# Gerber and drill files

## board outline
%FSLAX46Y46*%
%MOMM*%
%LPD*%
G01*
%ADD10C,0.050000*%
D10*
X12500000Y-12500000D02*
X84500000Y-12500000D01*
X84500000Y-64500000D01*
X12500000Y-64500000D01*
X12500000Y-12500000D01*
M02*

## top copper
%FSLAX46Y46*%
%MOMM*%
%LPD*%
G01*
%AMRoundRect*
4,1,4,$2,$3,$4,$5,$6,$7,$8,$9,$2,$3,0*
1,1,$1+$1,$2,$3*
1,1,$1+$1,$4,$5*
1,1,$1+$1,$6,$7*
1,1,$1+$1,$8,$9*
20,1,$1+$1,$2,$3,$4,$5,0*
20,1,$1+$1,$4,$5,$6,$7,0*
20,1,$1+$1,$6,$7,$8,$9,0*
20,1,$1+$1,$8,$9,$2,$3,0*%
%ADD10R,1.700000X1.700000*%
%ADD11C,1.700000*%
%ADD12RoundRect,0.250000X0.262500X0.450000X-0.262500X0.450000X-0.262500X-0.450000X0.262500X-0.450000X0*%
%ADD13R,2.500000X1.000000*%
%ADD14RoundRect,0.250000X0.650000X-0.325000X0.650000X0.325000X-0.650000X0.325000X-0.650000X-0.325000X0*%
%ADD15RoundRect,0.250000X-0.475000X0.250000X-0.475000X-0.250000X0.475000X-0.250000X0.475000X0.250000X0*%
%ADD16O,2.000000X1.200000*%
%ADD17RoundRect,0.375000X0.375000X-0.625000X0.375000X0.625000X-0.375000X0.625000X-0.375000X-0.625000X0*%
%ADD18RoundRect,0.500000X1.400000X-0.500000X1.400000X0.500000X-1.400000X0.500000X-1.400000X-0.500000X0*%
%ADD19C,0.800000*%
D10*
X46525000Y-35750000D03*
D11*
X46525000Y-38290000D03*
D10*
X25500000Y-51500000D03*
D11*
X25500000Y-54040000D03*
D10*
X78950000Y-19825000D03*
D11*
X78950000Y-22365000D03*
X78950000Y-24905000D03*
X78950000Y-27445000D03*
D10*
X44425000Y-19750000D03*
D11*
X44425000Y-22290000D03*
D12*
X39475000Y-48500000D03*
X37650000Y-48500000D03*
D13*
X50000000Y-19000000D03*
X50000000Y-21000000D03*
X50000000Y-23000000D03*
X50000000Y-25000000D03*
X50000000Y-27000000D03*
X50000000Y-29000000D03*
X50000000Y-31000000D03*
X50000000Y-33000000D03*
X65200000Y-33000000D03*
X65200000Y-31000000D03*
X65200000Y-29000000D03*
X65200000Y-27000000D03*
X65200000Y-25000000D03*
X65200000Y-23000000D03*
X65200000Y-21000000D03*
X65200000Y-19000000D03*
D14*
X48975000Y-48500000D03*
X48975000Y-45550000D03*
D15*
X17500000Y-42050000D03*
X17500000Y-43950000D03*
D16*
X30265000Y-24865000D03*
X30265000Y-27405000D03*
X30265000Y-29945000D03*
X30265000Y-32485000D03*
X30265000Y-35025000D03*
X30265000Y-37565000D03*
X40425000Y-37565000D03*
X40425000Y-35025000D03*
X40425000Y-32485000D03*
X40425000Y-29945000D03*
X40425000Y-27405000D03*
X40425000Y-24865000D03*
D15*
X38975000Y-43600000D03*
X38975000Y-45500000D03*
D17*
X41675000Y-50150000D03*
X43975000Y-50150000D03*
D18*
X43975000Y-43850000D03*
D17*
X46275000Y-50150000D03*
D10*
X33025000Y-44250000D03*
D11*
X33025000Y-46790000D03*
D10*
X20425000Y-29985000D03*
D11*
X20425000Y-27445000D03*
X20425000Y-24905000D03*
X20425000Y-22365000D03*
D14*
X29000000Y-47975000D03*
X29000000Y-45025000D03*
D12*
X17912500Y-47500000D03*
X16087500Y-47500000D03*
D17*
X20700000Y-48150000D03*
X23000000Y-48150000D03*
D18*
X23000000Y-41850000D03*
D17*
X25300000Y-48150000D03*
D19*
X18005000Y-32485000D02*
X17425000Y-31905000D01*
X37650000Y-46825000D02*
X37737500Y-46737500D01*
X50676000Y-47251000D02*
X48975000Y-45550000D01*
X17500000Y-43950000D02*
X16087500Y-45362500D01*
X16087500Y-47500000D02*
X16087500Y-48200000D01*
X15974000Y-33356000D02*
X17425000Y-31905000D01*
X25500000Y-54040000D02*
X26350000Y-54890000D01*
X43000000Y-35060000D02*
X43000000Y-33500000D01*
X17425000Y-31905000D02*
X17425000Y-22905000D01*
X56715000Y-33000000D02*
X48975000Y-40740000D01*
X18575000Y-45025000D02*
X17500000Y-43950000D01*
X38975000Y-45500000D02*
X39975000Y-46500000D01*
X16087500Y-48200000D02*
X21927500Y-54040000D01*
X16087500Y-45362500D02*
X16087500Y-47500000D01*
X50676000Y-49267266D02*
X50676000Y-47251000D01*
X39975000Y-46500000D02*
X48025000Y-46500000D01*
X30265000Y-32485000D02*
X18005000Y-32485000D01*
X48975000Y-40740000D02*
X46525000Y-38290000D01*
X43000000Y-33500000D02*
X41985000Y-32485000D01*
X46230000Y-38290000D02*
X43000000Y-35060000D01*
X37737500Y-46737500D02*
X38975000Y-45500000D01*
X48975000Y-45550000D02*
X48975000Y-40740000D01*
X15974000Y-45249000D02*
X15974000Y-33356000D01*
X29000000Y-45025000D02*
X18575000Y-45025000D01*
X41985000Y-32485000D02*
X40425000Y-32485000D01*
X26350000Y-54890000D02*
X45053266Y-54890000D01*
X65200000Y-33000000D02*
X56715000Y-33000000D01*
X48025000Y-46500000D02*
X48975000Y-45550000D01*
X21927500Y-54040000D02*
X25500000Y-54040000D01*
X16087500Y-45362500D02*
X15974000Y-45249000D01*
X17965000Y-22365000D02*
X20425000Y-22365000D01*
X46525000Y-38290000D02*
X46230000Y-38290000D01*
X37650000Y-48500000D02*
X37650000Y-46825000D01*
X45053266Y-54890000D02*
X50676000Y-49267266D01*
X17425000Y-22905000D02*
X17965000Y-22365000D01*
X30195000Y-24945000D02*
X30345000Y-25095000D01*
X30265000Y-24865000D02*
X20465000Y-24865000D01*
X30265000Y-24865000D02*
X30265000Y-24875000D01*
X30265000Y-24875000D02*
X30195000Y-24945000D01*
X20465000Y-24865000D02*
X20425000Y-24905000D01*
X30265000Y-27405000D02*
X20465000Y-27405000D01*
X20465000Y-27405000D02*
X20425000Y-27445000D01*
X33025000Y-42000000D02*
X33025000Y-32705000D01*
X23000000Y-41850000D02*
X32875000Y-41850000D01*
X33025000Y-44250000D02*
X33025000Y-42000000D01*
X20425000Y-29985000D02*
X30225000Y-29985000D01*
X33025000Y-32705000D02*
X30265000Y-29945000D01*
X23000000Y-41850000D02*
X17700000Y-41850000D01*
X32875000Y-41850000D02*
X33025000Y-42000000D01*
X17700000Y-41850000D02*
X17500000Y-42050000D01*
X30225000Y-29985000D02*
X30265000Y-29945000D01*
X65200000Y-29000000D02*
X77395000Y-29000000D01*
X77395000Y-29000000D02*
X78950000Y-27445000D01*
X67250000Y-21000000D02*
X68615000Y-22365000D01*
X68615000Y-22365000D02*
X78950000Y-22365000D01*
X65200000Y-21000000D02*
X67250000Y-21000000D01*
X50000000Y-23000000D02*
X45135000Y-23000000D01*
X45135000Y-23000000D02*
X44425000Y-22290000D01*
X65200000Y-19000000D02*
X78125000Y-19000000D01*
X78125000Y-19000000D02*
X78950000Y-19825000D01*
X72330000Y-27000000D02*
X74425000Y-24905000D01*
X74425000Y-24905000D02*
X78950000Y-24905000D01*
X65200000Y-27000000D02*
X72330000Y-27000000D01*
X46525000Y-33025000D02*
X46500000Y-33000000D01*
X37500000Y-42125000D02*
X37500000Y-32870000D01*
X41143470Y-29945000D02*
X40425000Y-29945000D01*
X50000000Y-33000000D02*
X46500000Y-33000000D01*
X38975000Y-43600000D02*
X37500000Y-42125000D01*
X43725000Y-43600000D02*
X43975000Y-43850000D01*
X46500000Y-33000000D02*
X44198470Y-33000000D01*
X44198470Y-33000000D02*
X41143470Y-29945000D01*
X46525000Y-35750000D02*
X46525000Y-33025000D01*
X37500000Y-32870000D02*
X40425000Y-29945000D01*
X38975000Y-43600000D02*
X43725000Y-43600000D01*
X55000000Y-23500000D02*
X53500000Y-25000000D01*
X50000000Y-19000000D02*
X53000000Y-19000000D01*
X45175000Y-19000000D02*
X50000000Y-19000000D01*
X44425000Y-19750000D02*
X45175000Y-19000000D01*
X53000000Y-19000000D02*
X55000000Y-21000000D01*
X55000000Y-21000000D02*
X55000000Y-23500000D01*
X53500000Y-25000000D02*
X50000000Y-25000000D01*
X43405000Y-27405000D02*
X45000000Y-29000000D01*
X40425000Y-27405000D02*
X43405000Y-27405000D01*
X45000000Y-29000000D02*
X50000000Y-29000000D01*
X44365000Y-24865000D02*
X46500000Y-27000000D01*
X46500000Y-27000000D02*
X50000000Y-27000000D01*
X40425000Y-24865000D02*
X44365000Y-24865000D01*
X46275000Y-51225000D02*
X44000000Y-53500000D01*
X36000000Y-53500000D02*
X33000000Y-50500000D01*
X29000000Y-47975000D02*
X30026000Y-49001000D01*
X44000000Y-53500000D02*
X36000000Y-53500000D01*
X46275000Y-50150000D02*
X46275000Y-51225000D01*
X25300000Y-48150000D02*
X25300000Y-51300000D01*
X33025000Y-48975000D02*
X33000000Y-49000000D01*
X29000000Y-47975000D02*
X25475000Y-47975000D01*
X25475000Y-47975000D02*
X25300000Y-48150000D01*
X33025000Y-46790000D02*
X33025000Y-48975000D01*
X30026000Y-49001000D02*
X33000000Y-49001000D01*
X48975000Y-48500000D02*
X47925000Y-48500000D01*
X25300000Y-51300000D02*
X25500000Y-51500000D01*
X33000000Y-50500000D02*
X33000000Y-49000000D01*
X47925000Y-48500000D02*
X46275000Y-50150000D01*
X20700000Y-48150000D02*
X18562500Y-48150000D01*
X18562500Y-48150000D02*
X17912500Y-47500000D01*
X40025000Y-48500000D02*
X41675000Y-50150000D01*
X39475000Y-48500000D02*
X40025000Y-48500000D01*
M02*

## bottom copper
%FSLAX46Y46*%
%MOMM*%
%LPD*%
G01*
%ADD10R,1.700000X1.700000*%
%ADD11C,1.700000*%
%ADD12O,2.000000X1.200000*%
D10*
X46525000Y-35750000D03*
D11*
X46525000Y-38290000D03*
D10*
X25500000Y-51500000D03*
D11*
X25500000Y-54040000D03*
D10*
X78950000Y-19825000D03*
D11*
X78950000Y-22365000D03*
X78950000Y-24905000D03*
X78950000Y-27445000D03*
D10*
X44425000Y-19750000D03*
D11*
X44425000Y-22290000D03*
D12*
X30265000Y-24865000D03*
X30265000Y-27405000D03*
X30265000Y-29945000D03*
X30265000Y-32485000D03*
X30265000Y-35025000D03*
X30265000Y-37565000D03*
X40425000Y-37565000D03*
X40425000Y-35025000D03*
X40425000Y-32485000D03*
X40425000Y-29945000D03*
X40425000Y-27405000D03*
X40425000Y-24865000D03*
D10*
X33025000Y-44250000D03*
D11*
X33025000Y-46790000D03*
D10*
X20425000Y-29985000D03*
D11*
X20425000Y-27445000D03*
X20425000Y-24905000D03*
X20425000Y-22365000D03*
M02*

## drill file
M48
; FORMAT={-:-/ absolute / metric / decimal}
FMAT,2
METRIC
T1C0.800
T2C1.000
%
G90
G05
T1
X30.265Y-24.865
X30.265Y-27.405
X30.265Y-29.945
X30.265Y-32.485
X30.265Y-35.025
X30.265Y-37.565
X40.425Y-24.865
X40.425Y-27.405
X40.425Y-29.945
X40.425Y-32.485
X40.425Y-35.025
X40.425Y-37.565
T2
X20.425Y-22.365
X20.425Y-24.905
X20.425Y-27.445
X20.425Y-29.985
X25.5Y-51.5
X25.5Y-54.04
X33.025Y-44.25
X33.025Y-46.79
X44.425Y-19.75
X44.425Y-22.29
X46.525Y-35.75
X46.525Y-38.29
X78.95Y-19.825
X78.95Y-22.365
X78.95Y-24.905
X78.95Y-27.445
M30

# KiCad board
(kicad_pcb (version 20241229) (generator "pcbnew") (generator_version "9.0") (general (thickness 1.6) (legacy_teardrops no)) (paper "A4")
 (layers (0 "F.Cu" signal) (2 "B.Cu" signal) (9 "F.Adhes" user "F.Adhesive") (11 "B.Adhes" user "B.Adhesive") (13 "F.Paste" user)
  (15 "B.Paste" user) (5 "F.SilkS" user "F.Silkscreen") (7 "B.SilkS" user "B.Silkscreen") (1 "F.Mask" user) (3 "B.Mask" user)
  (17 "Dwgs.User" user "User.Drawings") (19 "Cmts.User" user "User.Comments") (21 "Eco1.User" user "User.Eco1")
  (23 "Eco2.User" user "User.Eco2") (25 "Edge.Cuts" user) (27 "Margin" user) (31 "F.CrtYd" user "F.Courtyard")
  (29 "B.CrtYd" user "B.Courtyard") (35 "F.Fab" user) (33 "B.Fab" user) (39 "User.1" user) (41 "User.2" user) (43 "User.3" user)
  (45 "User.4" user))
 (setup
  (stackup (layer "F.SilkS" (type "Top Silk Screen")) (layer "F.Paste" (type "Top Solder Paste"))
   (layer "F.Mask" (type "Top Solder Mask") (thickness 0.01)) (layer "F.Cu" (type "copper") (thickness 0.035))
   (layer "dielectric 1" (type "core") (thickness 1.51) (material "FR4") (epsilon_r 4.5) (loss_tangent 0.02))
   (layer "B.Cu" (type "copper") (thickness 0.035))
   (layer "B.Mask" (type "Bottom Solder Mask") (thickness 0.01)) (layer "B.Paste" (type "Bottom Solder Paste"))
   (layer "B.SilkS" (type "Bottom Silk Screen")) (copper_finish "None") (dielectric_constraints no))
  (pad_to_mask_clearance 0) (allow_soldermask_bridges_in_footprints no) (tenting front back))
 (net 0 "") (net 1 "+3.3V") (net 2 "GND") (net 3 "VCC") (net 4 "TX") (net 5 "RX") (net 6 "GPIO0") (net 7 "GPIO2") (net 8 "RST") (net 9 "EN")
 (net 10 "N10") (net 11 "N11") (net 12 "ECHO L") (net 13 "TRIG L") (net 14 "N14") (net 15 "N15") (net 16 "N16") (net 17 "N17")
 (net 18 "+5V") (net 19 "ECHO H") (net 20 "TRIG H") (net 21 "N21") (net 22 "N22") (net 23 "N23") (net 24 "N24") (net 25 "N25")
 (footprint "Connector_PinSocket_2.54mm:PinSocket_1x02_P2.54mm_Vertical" (layer "F.Cu") (at 46.525 35.75)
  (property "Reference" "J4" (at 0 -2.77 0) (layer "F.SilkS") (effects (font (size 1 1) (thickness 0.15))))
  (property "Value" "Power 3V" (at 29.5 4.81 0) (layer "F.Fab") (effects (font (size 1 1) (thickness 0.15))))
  (pad "1" thru_hole rect (at 0 0) (size 1.7 1.7) (drill 1) (layers "*.Cu" "*.Mask") (remove_unused_layers no) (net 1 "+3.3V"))
  (pad "2" thru_hole circle (at 0 2.54) (size 1.7 1.7) (drill 1) (layers "*.Cu" "*.Mask") (remove_unused_layers no) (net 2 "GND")))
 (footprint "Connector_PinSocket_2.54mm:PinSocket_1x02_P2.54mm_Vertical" (layer "F.Cu") (at 25.5 51.5)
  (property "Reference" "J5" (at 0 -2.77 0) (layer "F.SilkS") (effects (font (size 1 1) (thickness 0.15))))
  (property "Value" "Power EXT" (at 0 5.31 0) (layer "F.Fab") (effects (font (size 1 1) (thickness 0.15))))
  (pad "1" thru_hole rect (at 0 0) (size 1.7 1.7) (drill 1) (layers "*.Cu" "*.Mask") (remove_unused_layers no) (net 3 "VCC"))
  (pad "2" thru_hole circle (at 0 2.54) (size 1.7 1.7) (drill 1) (layers "*.Cu" "*.Mask") (remove_unused_layers no) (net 2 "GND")))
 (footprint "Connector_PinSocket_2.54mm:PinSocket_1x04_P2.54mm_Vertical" (layer "F.Cu") (at 78.95 19.825)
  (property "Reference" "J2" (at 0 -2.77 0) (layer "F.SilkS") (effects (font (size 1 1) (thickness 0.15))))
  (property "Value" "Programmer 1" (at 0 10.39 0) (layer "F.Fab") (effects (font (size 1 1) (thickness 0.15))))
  (pad "1" thru_hole rect (at 0 0) (size 1.7 1.7) (drill 1) (layers "*.Cu" "*.Mask") (remove_unused_layers no) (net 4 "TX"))
  (pad "2" thru_hole circle (at 0 2.54) (size 1.7 1.7) (drill 1) (layers "*.Cu" "*.Mask") (remove_unused_layers no) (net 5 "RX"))
  (pad "3" thru_hole circle (at 0 5.08) (size 1.7 1.7) (drill 1) (layers "*.Cu" "*.Mask") (remove_unused_layers no) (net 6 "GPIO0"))
  (pad "4" thru_hole circle (at 0 7.62) (size 1.7 1.7) (drill 1) (layers "*.Cu" "*.Mask") (remove_unused_layers no) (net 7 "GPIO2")))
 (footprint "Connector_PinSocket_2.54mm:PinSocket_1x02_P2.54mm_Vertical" (layer "F.Cu") (at 44.425 19.75)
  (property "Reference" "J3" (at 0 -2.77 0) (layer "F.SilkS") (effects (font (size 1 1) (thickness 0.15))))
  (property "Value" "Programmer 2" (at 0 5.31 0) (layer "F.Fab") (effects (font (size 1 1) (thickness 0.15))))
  (pad "1" thru_hole rect (at 0 0) (size 1.7 1.7) (drill 1) (layers "*.Cu" "*.Mask") (remove_unused_layers no) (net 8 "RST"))
  (pad "2" thru_hole circle (at 0 2.54) (size 1.7 1.7) (drill 1) (layers "*.Cu" "*.Mask") (remove_unused_layers no) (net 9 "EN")))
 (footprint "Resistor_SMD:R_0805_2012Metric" (layer "F.Cu") (at 38.5625 48.5 180)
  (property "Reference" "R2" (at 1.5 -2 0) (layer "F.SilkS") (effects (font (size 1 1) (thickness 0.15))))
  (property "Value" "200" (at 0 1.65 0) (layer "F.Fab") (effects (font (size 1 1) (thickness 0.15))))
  (pad "1" smd roundrect (at -0.9125 0 180) (size 1.025 1.4) (layers "F.Cu" "F.Mask" "F.Paste") (roundrect_rratio 0.243902) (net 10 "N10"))
  (pad "2" smd roundrect (at 0.9125 0 180) (size 1.025 1.4) (layers "F.Cu" "F.Mask" "F.Paste") (roundrect_rratio 0.243902) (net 2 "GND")))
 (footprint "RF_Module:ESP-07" (layer "F.Cu") (at 57.6 23.9)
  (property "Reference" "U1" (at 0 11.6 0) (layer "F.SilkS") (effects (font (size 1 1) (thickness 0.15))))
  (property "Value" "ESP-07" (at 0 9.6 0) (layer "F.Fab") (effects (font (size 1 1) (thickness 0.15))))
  (pad "1" smd rect (at -7.6 -4.9) (size 2.5 1) (layers "F.Cu" "F.Mask" "F.Paste") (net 8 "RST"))
  (pad "2" smd rect (at -7.6 -2.9) (size 2.5 1) (layers "F.Cu" "F.Mask" "F.Paste") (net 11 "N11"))
  (pad "3" smd rect (at -7.6 -0.9) (size 2.5 1) (layers "F.Cu" "F.Mask" "F.Paste") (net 9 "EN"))
  (pad "4" smd rect (at -7.6 1.1) (size 2.5 1) (layers "F.Cu" "F.Mask" "F.Paste") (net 8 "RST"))
  (pad "5" smd rect (at -7.6 3.1) (size 2.5 1) (layers "F.Cu" "F.Mask" "F.Paste") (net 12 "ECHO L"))
  (pad "6" smd rect (at -7.6 5.1) (size 2.5 1) (layers "F.Cu" "F.Mask" "F.Paste") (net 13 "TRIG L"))
  (pad "7" smd rect (at -7.6 7.1) (size 2.5 1) (layers "F.Cu" "F.Mask" "F.Paste") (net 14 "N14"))
  (pad "8" smd rect (at -7.6 9.1) (size 2.5 1) (layers "F.Cu" "F.Mask" "F.Paste") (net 1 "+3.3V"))
  (pad "9" smd rect (at 7.6 9.1) (size 2.5 1) (layers "F.Cu" "F.Mask" "F.Paste") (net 2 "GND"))
  (pad "10" smd rect (at 7.6 7.1) (size 2.5 1) (layers "F.Cu" "F.Mask" "F.Paste") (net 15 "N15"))
  (pad "11" smd rect (at 7.6 5.1) (size 2.5 1) (layers "F.Cu" "F.Mask" "F.Paste") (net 7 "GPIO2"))
  (pad "12" smd rect (at 7.6 3.1) (size 2.5 1) (layers "F.Cu" "F.Mask" "F.Paste") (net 6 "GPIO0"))
  (pad "13" smd rect (at 7.6 1.1) (size 2.5 1) (layers "F.Cu" "F.Mask" "F.Paste") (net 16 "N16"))
  (pad "14" smd rect (at 7.6 -0.9) (size 2.5 1) (layers "F.Cu" "F.Mask" "F.Paste") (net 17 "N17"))
  (pad "15" smd rect (at 7.6 -2.9) (size 2.5 1) (layers "F.Cu" "F.Mask" "F.Paste") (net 5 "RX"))
  (pad "16" smd rect (at 7.6 -4.9) (size 2.5 1) (layers "F.Cu" "F.Mask" "F.Paste") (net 4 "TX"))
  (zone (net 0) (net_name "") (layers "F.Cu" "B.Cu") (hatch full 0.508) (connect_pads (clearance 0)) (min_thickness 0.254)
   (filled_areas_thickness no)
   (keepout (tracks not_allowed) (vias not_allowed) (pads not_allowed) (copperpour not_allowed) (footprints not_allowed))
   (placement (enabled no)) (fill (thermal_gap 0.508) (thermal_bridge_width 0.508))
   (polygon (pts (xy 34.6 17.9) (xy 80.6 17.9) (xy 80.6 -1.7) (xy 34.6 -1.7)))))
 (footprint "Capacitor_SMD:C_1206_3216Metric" (layer "F.Cu") (at 48.975 47.025 90)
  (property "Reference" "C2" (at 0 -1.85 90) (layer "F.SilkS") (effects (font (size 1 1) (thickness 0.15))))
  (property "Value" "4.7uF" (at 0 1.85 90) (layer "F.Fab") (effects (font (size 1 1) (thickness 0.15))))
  (pad "1" smd roundrect (at -1.475 0 90) (size 1.15 1.8) (layers "F.Cu" "F.Mask" "F.Paste") (roundrect_rratio 0.217391) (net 3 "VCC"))
  (pad "2" smd roundrect (at 1.475 0 90) (size 1.15 1.8) (layers "F.Cu" "F.Mask" "F.Paste") (roundrect_rratio 0.217391) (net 2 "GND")))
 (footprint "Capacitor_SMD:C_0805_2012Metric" (layer "F.Cu") (at 17.5 43 -90)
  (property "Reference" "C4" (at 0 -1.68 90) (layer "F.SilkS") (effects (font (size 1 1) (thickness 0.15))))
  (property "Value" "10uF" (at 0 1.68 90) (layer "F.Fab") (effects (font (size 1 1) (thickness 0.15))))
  (pad "1" smd roundrect (at -0.95 0 270) (size 1 1.45) (layers "F.Cu" "F.Mask" "F.Paste") (roundrect_rratio 0.25) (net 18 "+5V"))
  (pad "2" smd roundrect (at 0.95 0 270) (size 1 1.45) (layers "F.Cu" "F.Mask" "F.Paste") (roundrect_rratio 0.25) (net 2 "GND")))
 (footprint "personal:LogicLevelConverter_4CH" (layer "F.Cu") (at 35.345 31.215 -90)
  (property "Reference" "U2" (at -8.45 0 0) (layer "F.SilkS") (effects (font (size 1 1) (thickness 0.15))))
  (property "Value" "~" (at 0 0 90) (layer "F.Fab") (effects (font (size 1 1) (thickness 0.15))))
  (pad "1" thru_hole oval (at -6.35 5.08 270) (size 1.2 2) (drill 0.8) (layers "*.Cu" "*.Mask") (remove_unused_layers no) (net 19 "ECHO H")
   (thermal_bridge_angle 45))
  (pad "2" thru_hole oval (at -3.81 5.08 270) (size 1.2 2) (drill 0.8) (layers "*.Cu" "*.Mask") (remove_unused_layers no) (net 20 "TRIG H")
   (thermal_bridge_angle 45))
  (pad "3" thru_hole oval (at -1.27 5.08 270) (size 1.2 2) (drill 0.8) (layers "*.Cu" "*.Mask") (remove_unused_layers no) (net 18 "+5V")
   (thermal_bridge_angle 45))
  (pad "4" thru_hole oval (at 1.27 5.08 270) (size 1.2 2) (drill 0.8) (layers "*.Cu" "*.Mask") (remove_unused_layers no) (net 2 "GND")
   (thermal_bridge_angle 45))
  (pad "5" thru_hole oval (at 3.81 5.08 270) (size 1.2 2) (drill 0.8) (layers "*.Cu" "*.Mask") (remove_unused_layers no) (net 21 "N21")
   (thermal_bridge_angle 45))
  (pad "6" thru_hole oval (at 6.35 5.08 270) (size 1.2 2) (drill 0.8) (layers "*.Cu" "*.Mask") (remove_unused_layers no) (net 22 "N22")
   (thermal_bridge_angle 45))
  (pad "7" thru_hole oval (at 6.35 -5.08 270) (size 1.2 2) (drill 0.8) (layers "*.Cu" "*.Mask") (remove_unused_layers no) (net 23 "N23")
   (thermal_bridge_angle 45))
  (pad "8" thru_hole oval (at 3.81 -5.08 270) (size 1.2 2) (drill 0.8) (layers "*.Cu" "*.Mask") (remove_unused_layers no) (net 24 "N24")
   (thermal_bridge_angle 45))
  (pad "9" thru_hole oval (at 1.27 -5.08 270) (size 1.2 2) (drill 0.8) (layers "*.Cu" "*.Mask") (remove_unused_layers no) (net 2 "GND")
   (thermal_bridge_angle 45))
  (pad "10" thru_hole oval (at -1.27 -5.08 270) (size 1.2 2) (drill 0.8) (layers "*.Cu" "*.Mask") (remove_unused_layers no) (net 1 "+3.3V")
   (thermal_bridge_angle 45))
  (pad "11" thru_hole oval (at -3.81 -5.08 270) (size 1.2 2) (drill 0.8) (layers "*.Cu" "*.Mask") (remove_unused_layers no)
   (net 13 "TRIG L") (thermal_bridge_angle 45))
  (pad "12" thru_hole oval (at -6.35 -5.08 270) (size 1.2 2) (drill 0.8) (layers "*.Cu" "*.Mask") (remove_unused_layers no)
   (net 12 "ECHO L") (thermal_bridge_angle 45)))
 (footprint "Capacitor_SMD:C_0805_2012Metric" (layer "F.Cu") (at 38.975 44.55 -90)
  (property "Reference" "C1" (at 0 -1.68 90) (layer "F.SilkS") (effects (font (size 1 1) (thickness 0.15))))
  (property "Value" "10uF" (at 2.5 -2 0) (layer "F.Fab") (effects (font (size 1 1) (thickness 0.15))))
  (pad "1" smd roundrect (at -0.95 0 270) (size 1 1.45) (layers "F.Cu" "F.Mask" "F.Paste") (roundrect_rratio 0.25) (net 1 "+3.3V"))
  (pad "2" smd roundrect (at 0.95 0 270) (size 1 1.45) (layers "F.Cu" "F.Mask" "F.Paste") (roundrect_rratio 0.25) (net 2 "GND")))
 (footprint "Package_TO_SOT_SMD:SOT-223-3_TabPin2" (layer "F.Cu") (at 43.975 47 90)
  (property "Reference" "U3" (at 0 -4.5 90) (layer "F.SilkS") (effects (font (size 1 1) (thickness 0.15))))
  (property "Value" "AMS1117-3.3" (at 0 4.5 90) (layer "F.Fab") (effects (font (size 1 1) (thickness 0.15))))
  (pad "1" smd roundrect (at -3.15 -2.3 90) (size 2 1.5) (layers "F.Cu" "F.Mask" "F.Paste") (roundrect_rratio 0.25) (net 10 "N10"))
  (pad "2" smd roundrect (at -3.15 0 90) (size 2 1.5) (layers "F.Cu" "F.Mask" "F.Paste") (roundrect_rratio 0.25) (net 1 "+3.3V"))
  (pad "2" smd roundrect (at 3.15 0 90) (size 2 3.8) (layers "F.Cu" "F.Mask" "F.Paste") (roundrect_rratio 0.25) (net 1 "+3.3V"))
  (pad "3" smd roundrect (at -3.15 2.3 90) (size 2 1.5) (layers "F.Cu" "F.Mask" "F.Paste") (roundrect_rratio 0.25) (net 3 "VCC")))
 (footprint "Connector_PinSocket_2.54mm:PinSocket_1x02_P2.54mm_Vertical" (layer "F.Cu") (at 33.025 44.25)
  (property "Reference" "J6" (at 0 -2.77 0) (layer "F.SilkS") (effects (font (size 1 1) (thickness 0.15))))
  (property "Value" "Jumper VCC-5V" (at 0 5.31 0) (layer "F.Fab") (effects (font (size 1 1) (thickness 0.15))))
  (pad "1" thru_hole rect (at 0 0) (size 1.7 1.7) (drill 1) (layers "*.Cu" "*.Mask") (remove_unused_layers no) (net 18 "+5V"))
  (pad "2" thru_hole circle (at 0 2.54) (size 1.7 1.7) (drill 1) (layers "*.Cu" "*.Mask") (remove_unused_layers no) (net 3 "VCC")))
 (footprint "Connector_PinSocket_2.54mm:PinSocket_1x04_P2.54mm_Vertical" (layer "F.Cu") (at 20.425 29.985 180)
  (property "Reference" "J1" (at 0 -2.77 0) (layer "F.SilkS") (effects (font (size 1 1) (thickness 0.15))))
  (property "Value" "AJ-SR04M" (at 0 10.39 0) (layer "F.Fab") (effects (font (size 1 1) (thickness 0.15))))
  (pad "1" thru_hole rect (at 0 0 180) (size 1.7 1.7) (drill 1) (layers "*.Cu" "*.Mask") (remove_unused_layers no) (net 18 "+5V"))
  (pad "2" thru_hole circle (at 0 2.54 180) (size 1.7 1.7) (drill 1) (layers "*.Cu" "*.Mask") (remove_unused_layers no) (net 20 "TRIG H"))
  (pad "3" thru_hole circle (at 0 5.08 180) (size 1.7 1.7) (drill 1) (layers "*.Cu" "*.Mask") (remove_unused_layers no) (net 19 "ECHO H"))
  (pad "4" thru_hole circle (at 0 7.62 180) (size 1.7 1.7) (drill 1) (layers "*.Cu" "*.Mask") (remove_unused_layers no) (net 2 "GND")))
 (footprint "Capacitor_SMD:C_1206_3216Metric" (layer "F.Cu") (at 29 46.5 90)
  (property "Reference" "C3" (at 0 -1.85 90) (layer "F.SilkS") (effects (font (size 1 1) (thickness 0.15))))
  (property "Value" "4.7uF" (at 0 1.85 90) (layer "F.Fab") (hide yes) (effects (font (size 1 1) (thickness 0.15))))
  (pad "1" smd roundrect (at -1.475 0 90) (size 1.15 1.8) (layers "F.Cu" "F.Mask" "F.Paste") (roundrect_rratio 0.217391) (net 3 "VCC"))
  (pad "2" smd roundrect (at 1.475 0 90) (size 1.15 1.8) (layers "F.Cu" "F.Mask" "F.Paste") (roundrect_rratio 0.217391) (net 2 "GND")))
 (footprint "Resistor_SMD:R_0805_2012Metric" (layer "F.Cu") (at 17 47.5 180)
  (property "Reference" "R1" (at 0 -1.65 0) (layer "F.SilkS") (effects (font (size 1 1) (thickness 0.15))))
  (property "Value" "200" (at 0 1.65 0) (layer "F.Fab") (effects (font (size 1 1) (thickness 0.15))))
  (pad "1" smd roundrect (at -0.9125 0 180) (size 1.025 1.4) (layers "F.Cu" "F.Mask" "F.Paste") (roundrect_rratio 0.243902) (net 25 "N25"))
  (pad "2" smd roundrect (at 0.9125 0 180) (size 1.025 1.4) (layers "F.Cu" "F.Mask" "F.Paste") (roundrect_rratio 0.243902) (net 2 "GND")))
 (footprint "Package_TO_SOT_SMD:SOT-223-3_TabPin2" (layer "F.Cu") (at 23 45 90)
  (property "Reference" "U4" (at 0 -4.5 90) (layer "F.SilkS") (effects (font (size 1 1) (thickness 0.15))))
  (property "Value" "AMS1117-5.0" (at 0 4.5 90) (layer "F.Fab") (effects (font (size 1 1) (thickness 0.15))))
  (pad "1" smd roundrect (at -3.15 -2.3 90) (size 2 1.5) (layers "F.Cu" "F.Mask" "F.Paste") (roundrect_rratio 0.25) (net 25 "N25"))
  (pad "2" smd roundrect (at -3.15 0 90) (size 2 1.5) (layers "F.Cu" "F.Mask" "F.Paste") (roundrect_rratio 0.25) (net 18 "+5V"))
  (pad "2" smd roundrect (at 3.15 0 90) (size 2 3.8) (layers "F.Cu" "F.Mask" "F.Paste") (roundrect_rratio 0.25) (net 18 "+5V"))
  (pad "3" smd roundrect (at -3.15 2.3 90) (size 2 1.5) (layers "F.Cu" "F.Mask" "F.Paste") (roundrect_rratio 0.25) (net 3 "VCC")))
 (gr_rect (start 12.5 12.5) (end 84.5 64.5) (stroke (width 0.05) (type default)) (fill no) (layer "Edge.Cuts"))
 (segment (start 18.005 32.485) (end 17.425 31.905) (width 0.8) (layer "F.Cu") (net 2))
 (segment (start 37.65 46.825) (end 37.7375 46.7375) (width 0.8) (layer "F.Cu") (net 2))
 (segment (start 50.676 47.251) (end 48.975 45.55) (width 0.8) (layer "F.Cu") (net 2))
 (segment (start 17.5 43.95) (end 16.0875 45.3625) (width 0.8) (layer "F.Cu") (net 2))
 (segment (start 16.0875 47.5) (end 16.0875 48.2) (width 0.8) (layer "F.Cu") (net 2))
 (segment (start 15.974 33.356) (end 17.425 31.905) (width 0.8) (layer "F.Cu") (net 2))
 (segment (start 25.5 54.04) (end 26.35 54.89) (width 0.8) (layer "F.Cu") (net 2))
 (segment (start 43 35.06) (end 43 33.5) (width 0.8) (layer "F.Cu") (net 2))
 (segment (start 17.425 31.905) (end 17.425 22.905) (width 0.8) (layer "F.Cu") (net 2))
 (segment (start 56.715 33) (end 48.975 40.74) (width 0.8) (layer "F.Cu") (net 2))
 (segment (start 18.575 45.025) (end 17.5 43.95) (width 0.8) (layer "F.Cu") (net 2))
 (segment (start 38.975 45.5) (end 39.975 46.5) (width 0.8) (layer "F.Cu") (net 2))
 (segment (start 16.0875 48.2) (end 21.9275 54.04) (width 0.8) (layer "F.Cu") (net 2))
 (segment (start 16.0875 45.3625) (end 16.0875 47.5) (width 0.8) (layer "F.Cu") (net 2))
 (segment (start 50.676 49.267266) (end 50.676 47.251) (width 0.8) (layer "F.Cu") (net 2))
 (segment (start 39.975 46.5) (end 48.025 46.5) (width 0.8) (layer "F.Cu") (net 2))
 (segment (start 30.265 32.485) (end 18.005 32.485) (width 0.8) (layer "F.Cu") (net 2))
 (segment (start 48.975 40.74) (end 46.525 38.29) (width 0.8) (layer "F.Cu") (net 2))
 (segment (start 43 33.5) (end 41.985 32.485) (width 0.8) (layer "F.Cu") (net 2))
 (segment (start 46.23 38.29) (end 43 35.06) (width 0.8) (layer "F.Cu") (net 2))
 (segment (start 37.7375 46.7375) (end 38.975 45.5) (width 0.8) (layer "F.Cu") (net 2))
 (segment (start 48.975 45.55) (end 48.975 40.74) (width 0.8) (layer "F.Cu") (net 2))
 (segment (start 15.974 45.249) (end 15.974 33.356) (width 0.8) (layer "F.Cu") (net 2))
 (segment (start 29 45.025) (end 18.575 45.025) (width 0.8) (layer "F.Cu") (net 2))
 (segment (start 41.985 32.485) (end 40.425 32.485) (width 0.8) (layer "F.Cu") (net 2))
 (segment (start 26.35 54.89) (end 45.053266 54.89) (width 0.8) (layer "F.Cu") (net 2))
 (segment (start 65.2 33) (end 56.715 33) (width 0.8) (layer "F.Cu") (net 2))
 (segment (start 48.025 46.5) (end 48.975 45.55) (width 0.8) (layer "F.Cu") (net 2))
 (segment (start 21.9275 54.04) (end 25.5 54.04) (width 0.8) (layer "F.Cu") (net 2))
 (segment (start 16.0875 45.3625) (end 15.974 45.249) (width 0.8) (layer "F.Cu") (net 2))
 (segment (start 17.965 22.365) (end 20.425 22.365) (width 0.8) (layer "F.Cu") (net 2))
 (segment (start 46.525 38.29) (end 46.23 38.29) (width 0.8) (layer "F.Cu") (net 2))
 (segment (start 37.65 48.5) (end 37.65 46.825) (width 0.8) (layer "F.Cu") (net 2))
 (segment (start 45.053266 54.89) (end 50.676 49.267266) (width 0.8) (layer "F.Cu") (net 2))
 (segment (start 17.425 22.905) (end 17.965 22.365) (width 0.8) (layer "F.Cu") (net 2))
 (segment (start 30.195 24.945) (end 30.345 25.095) (width 0.8) (layer "F.Cu") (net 19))
 (segment (start 30.265 24.865) (end 20.465 24.865) (width 0.8) (layer "F.Cu") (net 19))
 (segment (start 30.265 24.865) (end 30.265 24.875) (width 0.8) (layer "F.Cu") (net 19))
 (segment (start 30.265 24.875) (end 30.195 24.945) (width 0.8) (layer "F.Cu") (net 19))
 (segment (start 20.465 24.865) (end 20.425 24.905) (width 0.8) (layer "F.Cu") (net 19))
 (segment (start 30.265 27.405) (end 20.465 27.405) (width 0.8) (layer "F.Cu") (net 20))
 (segment (start 20.465 27.405) (end 20.425 27.445) (width 0.8) (layer "F.Cu") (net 20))
 (segment (start 33.025 42) (end 33.025 32.705) (width 0.8) (layer "F.Cu") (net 18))
 (segment (start 23 41.85) (end 32.875 41.85) (width 0.8) (layer "F.Cu") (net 18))
 (segment (start 33.025 44.25) (end 33.025 42) (width 0.8) (layer "F.Cu") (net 18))
 (segment (start 20.425 29.985) (end 30.225 29.985) (width 0.8) (layer "F.Cu") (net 18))
 (segment (start 33.025 32.705) (end 30.265 29.945) (width 0.8) (layer "F.Cu") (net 18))
 (segment (start 23 41.85) (end 17.7 41.85) (width 0.8) (layer "F.Cu") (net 18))
 (segment (start 32.875 41.85) (end 33.025 42) (width 0.8) (layer "F.Cu") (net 18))
 (segment (start 17.7 41.85) (end 17.5 42.05) (width 0.8) (layer "F.Cu") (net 18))
 (segment (start 30.225 29.985) (end 30.265 29.945) (width 0.8) (layer "F.Cu") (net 18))
 (segment (start 65.2 29) (end 77.395 29) (width 0.8) (layer "F.Cu") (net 7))
 (segment (start 77.395 29) (end 78.95 27.445) (width 0.8) (layer "F.Cu") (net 7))
 (segment (start 67.25 21) (end 68.615 22.365) (width 0.8) (layer "F.Cu") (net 5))
 (segment (start 68.615 22.365) (end 78.95 22.365) (width 0.8) (layer "F.Cu") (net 5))
 (segment (start 65.2 21) (end 67.25 21) (width 0.8) (layer "F.Cu") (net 5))
 (segment (start 50 23) (end 45.135 23) (width 0.8) (layer "F.Cu") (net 9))
 (segment (start 45.135 23) (end 44.425 22.29) (width 0.8) (layer "F.Cu") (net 9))
 (segment (start 65.2 19) (end 78.125 19) (width 0.8) (layer "F.Cu") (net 4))
 (segment (start 78.125 19) (end 78.95 19.825) (width 0.8) (layer "F.Cu") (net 4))
 (segment (start 72.33 27) (end 74.425 24.905) (width 0.8) (layer "F.Cu") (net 6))
 (segment (start 74.425 24.905) (end 78.95 24.905) (width 0.8) (layer "F.Cu") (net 6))
 (segment (start 65.2 27) (end 72.33 27) (width 0.8) (layer "F.Cu") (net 6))
 (segment (start 46.525 33.025) (end 46.5 33) (width 0.8) (layer "F.Cu") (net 1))
 (segment (start 37.5 42.125) (end 37.5 32.87) (width 0.8) (layer "F.Cu") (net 1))
 (segment (start 41.14347 29.945) (end 40.425 29.945) (width 0.8) (layer "F.Cu") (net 1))
 (segment (start 50 33) (end 46.5 33) (width 0.8) (layer "F.Cu") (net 1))
 (segment (start 38.975 43.6) (end 37.5 42.125) (width 0.8) (layer "F.Cu") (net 1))
 (segment (start 43.725 43.6) (end 43.975 43.85) (width 0.8) (layer "F.Cu") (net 1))
 (segment (start 46.5 33) (end 44.19847 33) (width 0.8) (layer "F.Cu") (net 1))
 (segment (start 44.19847 33) (end 41.14347 29.945) (width 0.8) (layer "F.Cu") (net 1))
 (segment (start 46.525 35.75) (end 46.525 33.025) (width 0.8) (layer "F.Cu") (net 1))
 (segment (start 37.5 32.87) (end 40.425 29.945) (width 0.8) (layer "F.Cu") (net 1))
 (segment (start 38.975 43.6) (end 43.725 43.6) (width 0.8) (layer "F.Cu") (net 1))
 (segment (start 55 23.5) (end 53.5 25) (width 0.8) (layer "F.Cu") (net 8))
 (segment (start 50 19) (end 53 19) (width 0.8) (layer "F.Cu") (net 8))
 (segment (start 45.175 19) (end 50 19) (width 0.8) (layer "F.Cu") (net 8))
 (segment (start 44.425 19.75) (end 45.175 19) (width 0.8) (layer "F.Cu") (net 8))
 (segment (start 53 19) (end 55 21) (width 0.8) (layer "F.Cu") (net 8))
 (segment (start 55 21) (end 55 23.5) (width 0.8) (layer "F.Cu") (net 8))
 (segment (start 53.5 25) (end 50 25) (width 0.8) (layer "F.Cu") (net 8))
 (segment (start 43.405 27.405) (end 45 29) (width 0.8) (layer "F.Cu") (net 13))
 (segment (start 40.425 27.405) (end 43.405 27.405) (width 0.8) (layer "F.Cu") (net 13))
 (segment (start 45 29) (end 50 29) (width 0.8) (layer "F.Cu") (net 13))
 (segment (start 44.365 24.865) (end 46.5 27) (width 0.8) (layer "F.Cu") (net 12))
 (segment (start 46.5 27) (end 50 27) (width 0.8) (layer "F.Cu") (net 12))
 (segment (start 40.425 24.865) (end 44.365 24.865) (width 0.8) (layer "F.Cu") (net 12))
 (segment (start 46.275 51.225) (end 44 53.5) (width 0.8) (layer "F.Cu") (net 3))
 (segment (start 36 53.5) (end 33 50.5) (width 0.8) (layer "F.Cu") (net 3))
 (segment (start 29 47.975) (end 30.026 49.001) (width 0.8) (layer "F.Cu") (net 3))
 (segment (start 44 53.5) (end 36 53.5) (width 0.8) (layer "F.Cu") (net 3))
 (segment (start 46.275 50.15) (end 46.275 51.225) (width 0.8) (layer "F.Cu") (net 3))
 (segment (start 25.3 48.15) (end 25.3 51.3) (width 0.8) (layer "F.Cu") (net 3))
 (segment (start 33.025 48.975) (end 33 49) (width 0.8) (layer "F.Cu") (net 3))
 (segment (start 29 47.975) (end 25.475 47.975) (width 0.8) (layer "F.Cu") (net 3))
 (segment (start 25.475 47.975) (end 25.3 48.15) (width 0.8) (layer "F.Cu") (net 3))
 (segment (start 33.025 46.79) (end 33.025 48.975) (width 0.8) (layer "F.Cu") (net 3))
 (segment (start 30.026 49.001) (end 33 49.001) (width 0.8) (layer "F.Cu") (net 3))
 (segment (start 48.975 48.5) (end 47.925 48.5) (width 0.8) (layer "F.Cu") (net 3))
 (segment (start 25.3 51.3) (end 25.5 51.5) (width 0.8) (layer "F.Cu") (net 3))
 (segment (start 33 50.5) (end 33 49) (width 0.8) (layer "F.Cu") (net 3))
 (segment (start 47.925 48.5) (end 46.275 50.15) (width 0.8) (layer "F.Cu") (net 3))
 (segment (start 20.7 48.15) (end 18.5625 48.15) (width 0.8) (layer "F.Cu") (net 25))
 (segment (start 18.5625 48.15) (end 17.9125 47.5) (width 0.8) (layer "F.Cu") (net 25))
 (segment (start 40.025 48.5) (end 41.675 50.15) (width 0.8) (layer "F.Cu") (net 10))
 (segment (start 39.475 48.5) (end 40.025 48.5) (width 0.8) (layer "F.Cu") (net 10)))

